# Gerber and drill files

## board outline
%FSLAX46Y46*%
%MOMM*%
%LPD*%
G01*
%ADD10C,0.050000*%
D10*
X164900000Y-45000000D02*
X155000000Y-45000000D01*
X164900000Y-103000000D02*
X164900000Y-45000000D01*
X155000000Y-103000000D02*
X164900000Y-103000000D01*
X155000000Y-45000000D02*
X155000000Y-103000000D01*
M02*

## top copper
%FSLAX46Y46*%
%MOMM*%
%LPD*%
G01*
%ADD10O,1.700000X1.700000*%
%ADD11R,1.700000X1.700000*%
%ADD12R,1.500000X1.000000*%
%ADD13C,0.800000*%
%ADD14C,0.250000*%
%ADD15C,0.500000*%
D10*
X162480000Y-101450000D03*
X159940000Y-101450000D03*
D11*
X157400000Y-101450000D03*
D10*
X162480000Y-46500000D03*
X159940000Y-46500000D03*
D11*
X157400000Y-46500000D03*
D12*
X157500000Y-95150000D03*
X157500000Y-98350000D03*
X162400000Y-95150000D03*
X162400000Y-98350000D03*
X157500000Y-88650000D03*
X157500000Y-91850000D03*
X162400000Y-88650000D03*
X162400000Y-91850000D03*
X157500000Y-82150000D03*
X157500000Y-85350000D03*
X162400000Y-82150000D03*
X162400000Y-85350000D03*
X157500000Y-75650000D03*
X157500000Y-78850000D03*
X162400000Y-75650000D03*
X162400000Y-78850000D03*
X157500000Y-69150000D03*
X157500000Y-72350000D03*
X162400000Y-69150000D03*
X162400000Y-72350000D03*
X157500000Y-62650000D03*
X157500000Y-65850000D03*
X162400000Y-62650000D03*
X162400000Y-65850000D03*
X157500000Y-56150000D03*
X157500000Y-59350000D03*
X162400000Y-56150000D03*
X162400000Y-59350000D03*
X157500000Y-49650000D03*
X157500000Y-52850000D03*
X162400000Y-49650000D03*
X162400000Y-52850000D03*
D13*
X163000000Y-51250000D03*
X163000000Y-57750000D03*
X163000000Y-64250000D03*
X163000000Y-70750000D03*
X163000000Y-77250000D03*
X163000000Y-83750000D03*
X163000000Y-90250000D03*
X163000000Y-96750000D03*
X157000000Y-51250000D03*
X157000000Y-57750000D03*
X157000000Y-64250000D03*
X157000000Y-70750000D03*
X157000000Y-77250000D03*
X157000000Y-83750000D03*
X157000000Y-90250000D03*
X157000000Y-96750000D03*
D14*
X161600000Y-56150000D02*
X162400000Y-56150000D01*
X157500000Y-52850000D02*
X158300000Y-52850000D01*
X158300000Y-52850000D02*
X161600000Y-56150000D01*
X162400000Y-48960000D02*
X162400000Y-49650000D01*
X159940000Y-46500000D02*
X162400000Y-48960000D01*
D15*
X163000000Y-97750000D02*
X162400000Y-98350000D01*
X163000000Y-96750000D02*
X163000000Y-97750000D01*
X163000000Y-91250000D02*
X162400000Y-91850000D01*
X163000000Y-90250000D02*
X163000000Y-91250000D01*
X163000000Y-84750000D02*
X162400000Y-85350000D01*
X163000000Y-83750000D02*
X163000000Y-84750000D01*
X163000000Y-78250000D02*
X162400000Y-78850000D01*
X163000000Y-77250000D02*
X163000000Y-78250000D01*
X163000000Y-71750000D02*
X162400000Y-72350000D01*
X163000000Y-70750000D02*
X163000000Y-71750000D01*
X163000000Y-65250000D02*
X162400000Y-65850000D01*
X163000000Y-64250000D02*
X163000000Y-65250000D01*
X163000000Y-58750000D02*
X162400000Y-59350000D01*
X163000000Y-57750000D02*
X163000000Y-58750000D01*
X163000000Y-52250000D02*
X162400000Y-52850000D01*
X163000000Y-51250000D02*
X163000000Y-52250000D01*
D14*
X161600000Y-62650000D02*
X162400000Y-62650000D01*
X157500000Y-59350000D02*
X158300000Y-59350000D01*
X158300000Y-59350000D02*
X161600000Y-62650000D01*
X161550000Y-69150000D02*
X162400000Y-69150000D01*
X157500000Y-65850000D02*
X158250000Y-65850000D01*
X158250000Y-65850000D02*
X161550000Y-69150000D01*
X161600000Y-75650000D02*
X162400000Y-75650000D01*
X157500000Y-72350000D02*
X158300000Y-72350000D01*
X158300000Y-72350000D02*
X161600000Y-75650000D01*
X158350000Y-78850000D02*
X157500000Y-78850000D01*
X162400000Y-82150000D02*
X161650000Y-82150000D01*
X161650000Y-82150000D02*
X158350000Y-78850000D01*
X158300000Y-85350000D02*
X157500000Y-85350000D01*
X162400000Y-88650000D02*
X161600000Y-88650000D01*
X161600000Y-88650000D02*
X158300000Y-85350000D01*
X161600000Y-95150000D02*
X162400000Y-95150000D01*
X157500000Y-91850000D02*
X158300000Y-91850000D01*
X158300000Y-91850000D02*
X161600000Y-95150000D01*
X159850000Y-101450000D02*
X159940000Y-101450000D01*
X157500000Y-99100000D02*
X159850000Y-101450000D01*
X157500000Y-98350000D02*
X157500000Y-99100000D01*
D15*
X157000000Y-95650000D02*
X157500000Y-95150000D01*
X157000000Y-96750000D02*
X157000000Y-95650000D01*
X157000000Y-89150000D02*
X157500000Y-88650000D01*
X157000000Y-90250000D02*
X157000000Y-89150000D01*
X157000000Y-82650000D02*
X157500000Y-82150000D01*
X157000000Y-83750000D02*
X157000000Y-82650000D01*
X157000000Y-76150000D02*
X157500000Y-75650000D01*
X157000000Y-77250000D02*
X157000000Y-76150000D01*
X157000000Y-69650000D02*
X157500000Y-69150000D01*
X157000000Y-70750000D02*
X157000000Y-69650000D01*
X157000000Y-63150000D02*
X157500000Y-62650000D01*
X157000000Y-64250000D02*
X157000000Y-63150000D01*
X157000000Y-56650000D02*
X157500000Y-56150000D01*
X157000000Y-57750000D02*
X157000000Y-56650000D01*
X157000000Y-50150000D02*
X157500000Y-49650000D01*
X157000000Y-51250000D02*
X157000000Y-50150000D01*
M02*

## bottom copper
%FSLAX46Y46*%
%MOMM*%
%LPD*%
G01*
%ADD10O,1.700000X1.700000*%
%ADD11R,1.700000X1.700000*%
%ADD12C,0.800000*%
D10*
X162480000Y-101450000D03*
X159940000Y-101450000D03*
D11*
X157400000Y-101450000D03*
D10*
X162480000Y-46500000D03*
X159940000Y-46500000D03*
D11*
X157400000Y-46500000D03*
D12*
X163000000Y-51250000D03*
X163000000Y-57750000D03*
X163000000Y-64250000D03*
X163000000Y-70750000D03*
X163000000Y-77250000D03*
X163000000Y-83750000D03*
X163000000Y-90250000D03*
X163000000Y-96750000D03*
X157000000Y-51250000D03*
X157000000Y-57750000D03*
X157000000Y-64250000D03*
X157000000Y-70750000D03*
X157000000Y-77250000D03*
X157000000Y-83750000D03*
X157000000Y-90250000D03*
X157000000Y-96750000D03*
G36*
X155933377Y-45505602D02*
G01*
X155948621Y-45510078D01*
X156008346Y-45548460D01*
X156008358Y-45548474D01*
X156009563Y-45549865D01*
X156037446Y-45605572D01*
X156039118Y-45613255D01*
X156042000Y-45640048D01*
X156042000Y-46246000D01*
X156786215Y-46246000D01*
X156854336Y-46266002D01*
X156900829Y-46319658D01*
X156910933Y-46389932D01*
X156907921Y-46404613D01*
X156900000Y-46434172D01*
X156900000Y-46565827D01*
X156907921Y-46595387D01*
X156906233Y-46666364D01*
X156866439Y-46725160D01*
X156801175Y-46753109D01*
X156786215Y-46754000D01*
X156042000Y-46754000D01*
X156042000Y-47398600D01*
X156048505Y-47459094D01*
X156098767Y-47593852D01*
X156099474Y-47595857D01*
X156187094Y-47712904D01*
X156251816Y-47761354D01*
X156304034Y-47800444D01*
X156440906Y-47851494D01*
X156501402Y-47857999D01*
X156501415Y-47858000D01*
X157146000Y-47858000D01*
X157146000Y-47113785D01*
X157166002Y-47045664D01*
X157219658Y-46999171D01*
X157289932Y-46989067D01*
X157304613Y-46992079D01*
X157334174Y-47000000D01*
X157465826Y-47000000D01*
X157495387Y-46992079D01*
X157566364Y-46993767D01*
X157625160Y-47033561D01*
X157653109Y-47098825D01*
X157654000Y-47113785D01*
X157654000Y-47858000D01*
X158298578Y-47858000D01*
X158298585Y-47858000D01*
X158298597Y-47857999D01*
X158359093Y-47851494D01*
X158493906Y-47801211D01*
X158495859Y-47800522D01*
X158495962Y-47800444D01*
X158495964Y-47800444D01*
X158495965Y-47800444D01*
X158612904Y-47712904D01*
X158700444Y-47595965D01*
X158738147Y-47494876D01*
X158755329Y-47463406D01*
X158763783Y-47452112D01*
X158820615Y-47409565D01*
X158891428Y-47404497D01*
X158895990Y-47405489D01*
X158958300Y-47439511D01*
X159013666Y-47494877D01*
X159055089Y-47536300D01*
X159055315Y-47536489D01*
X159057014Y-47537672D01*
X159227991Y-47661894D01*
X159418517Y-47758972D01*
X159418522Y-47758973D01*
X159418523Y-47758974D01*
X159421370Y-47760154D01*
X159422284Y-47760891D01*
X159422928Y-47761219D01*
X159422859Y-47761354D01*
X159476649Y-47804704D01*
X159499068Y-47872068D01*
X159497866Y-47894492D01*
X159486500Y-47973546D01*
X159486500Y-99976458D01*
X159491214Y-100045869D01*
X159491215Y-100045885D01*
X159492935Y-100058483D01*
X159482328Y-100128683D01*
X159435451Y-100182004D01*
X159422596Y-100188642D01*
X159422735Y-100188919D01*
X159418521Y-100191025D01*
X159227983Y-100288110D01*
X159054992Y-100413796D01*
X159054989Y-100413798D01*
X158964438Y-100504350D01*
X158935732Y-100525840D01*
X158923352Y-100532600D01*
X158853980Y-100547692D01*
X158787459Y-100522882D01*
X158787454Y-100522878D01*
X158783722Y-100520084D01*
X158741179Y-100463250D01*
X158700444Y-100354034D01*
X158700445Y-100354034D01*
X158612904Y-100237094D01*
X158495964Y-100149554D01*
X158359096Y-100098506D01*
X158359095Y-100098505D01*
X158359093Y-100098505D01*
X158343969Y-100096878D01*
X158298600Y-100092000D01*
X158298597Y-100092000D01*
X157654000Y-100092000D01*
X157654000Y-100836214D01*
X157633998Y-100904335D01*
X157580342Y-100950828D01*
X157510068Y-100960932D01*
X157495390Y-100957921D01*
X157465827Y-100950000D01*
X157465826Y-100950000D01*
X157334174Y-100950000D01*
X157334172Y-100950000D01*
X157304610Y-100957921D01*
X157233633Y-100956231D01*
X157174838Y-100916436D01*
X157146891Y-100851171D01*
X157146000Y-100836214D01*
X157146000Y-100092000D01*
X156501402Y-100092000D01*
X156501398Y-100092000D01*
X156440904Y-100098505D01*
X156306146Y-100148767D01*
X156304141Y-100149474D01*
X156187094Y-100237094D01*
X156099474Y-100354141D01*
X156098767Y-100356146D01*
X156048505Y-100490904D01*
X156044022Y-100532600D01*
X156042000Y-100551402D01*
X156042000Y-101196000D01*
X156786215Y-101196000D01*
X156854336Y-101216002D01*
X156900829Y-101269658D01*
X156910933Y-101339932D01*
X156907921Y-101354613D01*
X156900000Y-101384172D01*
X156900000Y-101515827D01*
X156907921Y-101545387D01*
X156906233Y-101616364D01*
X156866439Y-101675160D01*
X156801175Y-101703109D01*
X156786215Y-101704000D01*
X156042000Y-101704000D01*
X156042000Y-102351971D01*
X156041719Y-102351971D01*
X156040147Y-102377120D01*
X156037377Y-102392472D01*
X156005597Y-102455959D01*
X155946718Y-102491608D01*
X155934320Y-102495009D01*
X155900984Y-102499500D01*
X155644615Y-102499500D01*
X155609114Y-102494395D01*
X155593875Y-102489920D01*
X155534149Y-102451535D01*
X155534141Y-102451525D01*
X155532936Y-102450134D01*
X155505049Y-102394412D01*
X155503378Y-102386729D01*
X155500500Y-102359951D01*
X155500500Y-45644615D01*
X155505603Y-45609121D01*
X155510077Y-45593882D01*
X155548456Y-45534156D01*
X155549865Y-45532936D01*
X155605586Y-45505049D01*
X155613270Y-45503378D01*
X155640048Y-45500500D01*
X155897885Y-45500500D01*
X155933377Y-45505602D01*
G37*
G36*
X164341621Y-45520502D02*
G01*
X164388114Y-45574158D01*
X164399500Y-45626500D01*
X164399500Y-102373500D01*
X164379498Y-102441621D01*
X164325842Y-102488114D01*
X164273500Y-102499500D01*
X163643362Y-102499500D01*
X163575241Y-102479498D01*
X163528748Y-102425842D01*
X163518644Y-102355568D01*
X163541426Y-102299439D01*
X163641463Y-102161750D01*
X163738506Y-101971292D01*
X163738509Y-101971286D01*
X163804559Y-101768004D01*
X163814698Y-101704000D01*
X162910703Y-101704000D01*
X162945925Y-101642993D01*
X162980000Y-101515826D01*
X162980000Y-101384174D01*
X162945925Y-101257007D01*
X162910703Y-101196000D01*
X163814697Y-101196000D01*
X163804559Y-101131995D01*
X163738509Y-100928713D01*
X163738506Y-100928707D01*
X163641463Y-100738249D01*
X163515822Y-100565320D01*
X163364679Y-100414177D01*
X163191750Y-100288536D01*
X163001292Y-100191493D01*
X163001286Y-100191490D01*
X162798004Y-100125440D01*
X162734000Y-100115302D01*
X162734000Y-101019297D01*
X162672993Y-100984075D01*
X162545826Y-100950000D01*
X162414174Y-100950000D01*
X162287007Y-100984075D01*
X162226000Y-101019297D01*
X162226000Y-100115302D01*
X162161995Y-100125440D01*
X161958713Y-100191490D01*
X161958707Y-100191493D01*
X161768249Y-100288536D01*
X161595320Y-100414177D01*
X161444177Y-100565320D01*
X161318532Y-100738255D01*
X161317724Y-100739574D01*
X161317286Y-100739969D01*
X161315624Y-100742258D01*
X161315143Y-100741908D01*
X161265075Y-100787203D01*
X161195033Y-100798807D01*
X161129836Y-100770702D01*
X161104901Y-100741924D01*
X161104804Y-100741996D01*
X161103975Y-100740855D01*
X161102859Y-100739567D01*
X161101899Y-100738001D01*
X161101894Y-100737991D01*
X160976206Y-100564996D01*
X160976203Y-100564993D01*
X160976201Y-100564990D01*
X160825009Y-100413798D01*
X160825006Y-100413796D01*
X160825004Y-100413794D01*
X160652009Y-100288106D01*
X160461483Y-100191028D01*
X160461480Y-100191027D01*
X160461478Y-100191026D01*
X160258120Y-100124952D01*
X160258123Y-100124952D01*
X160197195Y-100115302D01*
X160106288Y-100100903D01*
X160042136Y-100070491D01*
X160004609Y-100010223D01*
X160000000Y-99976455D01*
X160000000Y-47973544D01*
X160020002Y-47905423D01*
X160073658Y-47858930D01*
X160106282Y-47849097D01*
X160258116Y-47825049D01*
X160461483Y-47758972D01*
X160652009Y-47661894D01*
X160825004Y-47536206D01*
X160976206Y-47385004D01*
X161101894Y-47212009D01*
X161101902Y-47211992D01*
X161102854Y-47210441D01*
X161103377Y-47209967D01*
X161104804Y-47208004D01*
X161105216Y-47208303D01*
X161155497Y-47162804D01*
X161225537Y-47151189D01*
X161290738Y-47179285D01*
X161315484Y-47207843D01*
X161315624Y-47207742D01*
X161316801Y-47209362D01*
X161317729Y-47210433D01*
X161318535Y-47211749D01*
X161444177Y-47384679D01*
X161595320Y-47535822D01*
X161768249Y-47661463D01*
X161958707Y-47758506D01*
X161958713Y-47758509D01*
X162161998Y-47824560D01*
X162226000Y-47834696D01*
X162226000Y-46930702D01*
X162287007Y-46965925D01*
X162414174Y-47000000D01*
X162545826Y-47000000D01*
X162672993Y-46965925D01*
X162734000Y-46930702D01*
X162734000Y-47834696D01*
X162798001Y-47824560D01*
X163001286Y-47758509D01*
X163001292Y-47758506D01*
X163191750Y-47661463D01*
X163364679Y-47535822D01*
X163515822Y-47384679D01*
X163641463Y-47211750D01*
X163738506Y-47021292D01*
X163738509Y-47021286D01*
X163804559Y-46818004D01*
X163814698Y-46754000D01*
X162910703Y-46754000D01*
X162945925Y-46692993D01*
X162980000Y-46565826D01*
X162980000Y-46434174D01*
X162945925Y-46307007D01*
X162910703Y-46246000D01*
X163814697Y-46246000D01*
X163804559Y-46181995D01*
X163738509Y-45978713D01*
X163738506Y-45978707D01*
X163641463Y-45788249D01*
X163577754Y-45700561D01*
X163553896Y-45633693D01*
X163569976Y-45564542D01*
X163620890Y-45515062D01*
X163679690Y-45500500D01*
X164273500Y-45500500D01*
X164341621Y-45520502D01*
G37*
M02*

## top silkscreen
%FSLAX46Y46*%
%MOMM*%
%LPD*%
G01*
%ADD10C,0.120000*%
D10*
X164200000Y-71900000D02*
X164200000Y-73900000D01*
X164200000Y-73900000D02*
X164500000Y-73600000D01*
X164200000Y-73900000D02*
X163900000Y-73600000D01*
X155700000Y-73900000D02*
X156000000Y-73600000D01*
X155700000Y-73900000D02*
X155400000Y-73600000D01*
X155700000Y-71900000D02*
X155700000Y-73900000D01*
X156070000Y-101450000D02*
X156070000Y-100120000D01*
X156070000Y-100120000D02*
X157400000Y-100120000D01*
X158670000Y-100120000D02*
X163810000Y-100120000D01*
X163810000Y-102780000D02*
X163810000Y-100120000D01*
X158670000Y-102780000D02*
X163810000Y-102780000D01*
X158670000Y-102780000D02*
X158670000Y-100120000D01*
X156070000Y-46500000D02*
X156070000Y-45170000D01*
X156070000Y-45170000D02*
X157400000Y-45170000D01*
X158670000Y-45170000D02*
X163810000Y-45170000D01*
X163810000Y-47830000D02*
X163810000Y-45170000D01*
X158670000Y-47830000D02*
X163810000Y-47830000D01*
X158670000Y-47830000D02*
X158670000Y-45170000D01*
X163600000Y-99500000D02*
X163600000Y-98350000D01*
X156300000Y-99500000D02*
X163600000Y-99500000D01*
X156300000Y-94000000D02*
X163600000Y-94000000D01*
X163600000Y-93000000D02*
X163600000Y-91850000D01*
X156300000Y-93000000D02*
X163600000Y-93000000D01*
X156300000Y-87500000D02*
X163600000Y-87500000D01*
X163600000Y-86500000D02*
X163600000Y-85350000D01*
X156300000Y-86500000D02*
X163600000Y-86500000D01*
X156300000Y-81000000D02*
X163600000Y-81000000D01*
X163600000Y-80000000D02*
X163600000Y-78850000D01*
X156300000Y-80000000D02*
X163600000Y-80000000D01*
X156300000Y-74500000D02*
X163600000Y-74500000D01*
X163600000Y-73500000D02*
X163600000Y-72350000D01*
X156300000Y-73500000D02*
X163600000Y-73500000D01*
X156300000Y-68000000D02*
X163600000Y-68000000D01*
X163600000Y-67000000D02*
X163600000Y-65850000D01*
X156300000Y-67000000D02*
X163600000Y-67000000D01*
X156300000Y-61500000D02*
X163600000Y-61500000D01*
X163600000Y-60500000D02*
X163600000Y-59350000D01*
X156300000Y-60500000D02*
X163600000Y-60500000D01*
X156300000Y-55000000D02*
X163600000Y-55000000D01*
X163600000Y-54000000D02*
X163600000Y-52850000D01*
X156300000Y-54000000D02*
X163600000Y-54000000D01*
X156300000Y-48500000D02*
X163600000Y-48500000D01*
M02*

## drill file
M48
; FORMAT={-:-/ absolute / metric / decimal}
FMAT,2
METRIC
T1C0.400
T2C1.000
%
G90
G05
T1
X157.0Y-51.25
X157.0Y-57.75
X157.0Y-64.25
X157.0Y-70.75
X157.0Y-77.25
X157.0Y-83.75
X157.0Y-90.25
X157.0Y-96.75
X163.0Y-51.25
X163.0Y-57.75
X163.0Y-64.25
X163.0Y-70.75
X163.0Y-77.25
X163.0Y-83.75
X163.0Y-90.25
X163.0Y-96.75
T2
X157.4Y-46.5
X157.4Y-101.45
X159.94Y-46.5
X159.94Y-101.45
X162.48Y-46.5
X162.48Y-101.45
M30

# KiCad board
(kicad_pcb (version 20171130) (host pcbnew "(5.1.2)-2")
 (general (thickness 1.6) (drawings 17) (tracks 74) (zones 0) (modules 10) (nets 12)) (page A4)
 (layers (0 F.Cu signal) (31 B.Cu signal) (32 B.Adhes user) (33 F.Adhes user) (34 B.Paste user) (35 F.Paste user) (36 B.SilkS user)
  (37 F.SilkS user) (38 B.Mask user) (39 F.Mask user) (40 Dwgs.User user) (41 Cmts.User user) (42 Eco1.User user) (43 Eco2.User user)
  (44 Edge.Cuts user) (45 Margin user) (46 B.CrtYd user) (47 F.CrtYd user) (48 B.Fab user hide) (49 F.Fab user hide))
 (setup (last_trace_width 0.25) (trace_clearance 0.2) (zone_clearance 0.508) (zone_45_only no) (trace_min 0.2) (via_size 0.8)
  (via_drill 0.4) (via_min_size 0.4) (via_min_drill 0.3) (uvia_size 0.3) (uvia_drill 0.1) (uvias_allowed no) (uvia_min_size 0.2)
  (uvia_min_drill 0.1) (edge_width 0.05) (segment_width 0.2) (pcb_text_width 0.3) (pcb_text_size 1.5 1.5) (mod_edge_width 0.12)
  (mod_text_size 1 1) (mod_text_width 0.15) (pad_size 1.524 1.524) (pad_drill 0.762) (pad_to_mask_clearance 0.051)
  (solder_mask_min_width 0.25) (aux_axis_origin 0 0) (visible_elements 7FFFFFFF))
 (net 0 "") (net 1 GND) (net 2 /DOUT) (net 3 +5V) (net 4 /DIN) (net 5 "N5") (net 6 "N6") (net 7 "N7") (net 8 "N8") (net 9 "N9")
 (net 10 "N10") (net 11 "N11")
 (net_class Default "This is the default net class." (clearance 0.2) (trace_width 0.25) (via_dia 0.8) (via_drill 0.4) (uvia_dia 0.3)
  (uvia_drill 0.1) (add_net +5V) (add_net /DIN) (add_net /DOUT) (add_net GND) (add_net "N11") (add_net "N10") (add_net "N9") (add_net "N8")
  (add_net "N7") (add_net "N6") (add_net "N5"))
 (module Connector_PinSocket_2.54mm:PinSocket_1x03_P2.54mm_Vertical (layer F.Cu) (at 157.4 101.45 90)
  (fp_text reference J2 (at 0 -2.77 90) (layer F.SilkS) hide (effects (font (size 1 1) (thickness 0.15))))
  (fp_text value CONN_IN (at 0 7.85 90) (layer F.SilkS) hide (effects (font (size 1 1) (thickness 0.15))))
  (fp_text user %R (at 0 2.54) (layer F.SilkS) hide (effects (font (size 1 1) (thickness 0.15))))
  (fp_line (start 0 -1.33) (end 1.33 -1.33) (layer F.SilkS) (width 0.12))
  (fp_line (start 1.33 -1.33) (end 1.33 0) (layer F.SilkS) (width 0.12))
  (fp_line (start 1.33 1.27) (end 1.33 6.41) (layer F.SilkS) (width 0.12))
  (fp_line (start -1.33 6.41) (end 1.33 6.41) (layer F.SilkS) (width 0.12))
  (fp_line (start -1.33 1.27) (end -1.33 6.41) (layer F.SilkS) (width 0.12))
  (fp_line (start -1.33 1.27) (end 1.33 1.27) (layer F.SilkS) (width 0.12))
  (pad 3 thru_hole oval (at 0 5.08 90) (size 1.7 1.7) (drill 1) (layers *.Cu *.Mask) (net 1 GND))
  (pad 2 thru_hole oval (at 0 2.54 90) (size 1.7 1.7) (drill 1) (layers *.Cu *.Mask) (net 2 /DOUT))
  (pad 1 thru_hole rect (at 0 0 90) (size 1.7 1.7) (drill 1) (layers *.Cu *.Mask) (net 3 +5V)))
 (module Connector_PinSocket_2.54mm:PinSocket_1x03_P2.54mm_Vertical (layer F.Cu) (at 157.4 46.5 90)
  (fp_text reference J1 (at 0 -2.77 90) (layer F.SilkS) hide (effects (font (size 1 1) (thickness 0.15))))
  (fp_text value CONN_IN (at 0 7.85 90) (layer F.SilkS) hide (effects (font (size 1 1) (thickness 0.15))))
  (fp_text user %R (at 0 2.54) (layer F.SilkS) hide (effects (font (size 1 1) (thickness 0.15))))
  (fp_line (start 0 -1.33) (end 1.33 -1.33) (layer F.SilkS) (width 0.12))
  (fp_line (start 1.33 -1.33) (end 1.33 0) (layer F.SilkS) (width 0.12))
  (fp_line (start 1.33 1.27) (end 1.33 6.41) (layer F.SilkS) (width 0.12))
  (fp_line (start -1.33 6.41) (end 1.33 6.41) (layer F.SilkS) (width 0.12))
  (fp_line (start -1.33 1.27) (end -1.33 6.41) (layer F.SilkS) (width 0.12))
  (fp_line (start -1.33 1.27) (end 1.33 1.27) (layer F.SilkS) (width 0.12))
  (pad 3 thru_hole oval (at 0 5.08 90) (size 1.7 1.7) (drill 1) (layers *.Cu *.Mask) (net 1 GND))
  (pad 2 thru_hole oval (at 0 2.54 90) (size 1.7 1.7) (drill 1) (layers *.Cu *.Mask) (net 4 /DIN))
  (pad 1 thru_hole rect (at 0 0 90) (size 1.7 1.7) (drill 1) (layers *.Cu *.Mask) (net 3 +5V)))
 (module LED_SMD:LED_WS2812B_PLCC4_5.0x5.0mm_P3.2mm (layer F.Cu) (at 159.95 96.75)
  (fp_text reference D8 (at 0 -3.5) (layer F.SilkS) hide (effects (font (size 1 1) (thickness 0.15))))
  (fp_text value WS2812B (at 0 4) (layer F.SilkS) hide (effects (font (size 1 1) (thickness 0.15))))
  (fp_line (start 3.65 2.75) (end 3.65 1.6) (layer F.SilkS) (width 0.12))
  (fp_line (start -3.65 2.75) (end 3.65 2.75) (layer F.SilkS) (width 0.12))
  (fp_line (start -3.65 -2.75) (end 3.65 -2.75) (layer F.SilkS) (width 0.12))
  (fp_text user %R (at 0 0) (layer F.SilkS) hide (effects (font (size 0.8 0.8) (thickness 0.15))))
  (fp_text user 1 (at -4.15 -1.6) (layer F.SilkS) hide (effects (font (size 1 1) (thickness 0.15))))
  (pad 1 smd rect (at -2.45 -1.6) (size 1.5 1) (layers F.Cu F.Paste F.Mask) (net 3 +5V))
  (pad 2 smd rect (at -2.45 1.6) (size 1.5 1) (layers F.Cu F.Paste F.Mask) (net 2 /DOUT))
  (pad 4 smd rect (at 2.45 -1.6) (size 1.5 1) (layers F.Cu F.Paste F.Mask) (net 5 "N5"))
  (pad 3 smd rect (at 2.45 1.6) (size 1.5 1) (layers F.Cu F.Paste F.Mask) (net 1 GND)))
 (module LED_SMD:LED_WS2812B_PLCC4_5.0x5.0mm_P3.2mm (layer F.Cu) (at 159.95 90.25)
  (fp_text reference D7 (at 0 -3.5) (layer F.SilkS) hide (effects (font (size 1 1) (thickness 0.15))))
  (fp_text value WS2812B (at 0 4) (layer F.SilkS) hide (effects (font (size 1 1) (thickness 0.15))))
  (fp_line (start 3.65 2.75) (end 3.65 1.6) (layer F.SilkS) (width 0.12))
  (fp_line (start -3.65 2.75) (end 3.65 2.75) (layer F.SilkS) (width 0.12))
  (fp_line (start -3.65 -2.75) (end 3.65 -2.75) (layer F.SilkS) (width 0.12))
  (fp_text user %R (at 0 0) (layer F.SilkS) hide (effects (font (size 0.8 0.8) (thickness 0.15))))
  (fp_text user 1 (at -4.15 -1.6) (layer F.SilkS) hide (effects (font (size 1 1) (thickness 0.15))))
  (pad 1 smd rect (at -2.45 -1.6) (size 1.5 1) (layers F.Cu F.Paste F.Mask) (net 3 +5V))
  (pad 2 smd rect (at -2.45 1.6) (size 1.5 1) (layers F.Cu F.Paste F.Mask) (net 5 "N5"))
  (pad 4 smd rect (at 2.45 -1.6) (size 1.5 1) (layers F.Cu F.Paste F.Mask) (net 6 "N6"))
  (pad 3 smd rect (at 2.45 1.6) (size 1.5 1) (layers F.Cu F.Paste F.Mask) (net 1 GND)))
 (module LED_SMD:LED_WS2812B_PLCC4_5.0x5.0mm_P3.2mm (layer F.Cu) (at 159.95 83.75)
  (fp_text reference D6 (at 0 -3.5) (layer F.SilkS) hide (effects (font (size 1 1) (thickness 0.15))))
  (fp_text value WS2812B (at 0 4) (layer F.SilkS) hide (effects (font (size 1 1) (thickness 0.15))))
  (fp_line (start 3.65 2.75) (end 3.65 1.6) (layer F.SilkS) (width 0.12))
  (fp_line (start -3.65 2.75) (end 3.65 2.75) (layer F.SilkS) (width 0.12))
  (fp_line (start -3.65 -2.75) (end 3.65 -2.75) (layer F.SilkS) (width 0.12))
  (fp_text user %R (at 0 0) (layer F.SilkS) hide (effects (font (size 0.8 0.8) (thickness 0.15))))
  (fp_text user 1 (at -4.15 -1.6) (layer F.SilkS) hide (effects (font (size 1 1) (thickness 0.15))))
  (pad 1 smd rect (at -2.45 -1.6) (size 1.5 1) (layers F.Cu F.Paste F.Mask) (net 3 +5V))
  (pad 2 smd rect (at -2.45 1.6) (size 1.5 1) (layers F.Cu F.Paste F.Mask) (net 6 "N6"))
  (pad 4 smd rect (at 2.45 -1.6) (size 1.5 1) (layers F.Cu F.Paste F.Mask) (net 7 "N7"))
  (pad 3 smd rect (at 2.45 1.6) (size 1.5 1) (layers F.Cu F.Paste F.Mask) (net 1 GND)))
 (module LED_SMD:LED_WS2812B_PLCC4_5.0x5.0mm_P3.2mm (layer F.Cu) (at 159.95 77.25)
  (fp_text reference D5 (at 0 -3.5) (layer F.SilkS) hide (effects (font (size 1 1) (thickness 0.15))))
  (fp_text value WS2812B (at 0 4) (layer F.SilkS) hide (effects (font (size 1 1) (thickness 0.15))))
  (fp_line (start 3.65 2.75) (end 3.65 1.6) (layer F.SilkS) (width 0.12))
  (fp_line (start -3.65 2.75) (end 3.65 2.75) (layer F.SilkS) (width 0.12))
  (fp_line (start -3.65 -2.75) (end 3.65 -2.75) (layer F.SilkS) (width 0.12))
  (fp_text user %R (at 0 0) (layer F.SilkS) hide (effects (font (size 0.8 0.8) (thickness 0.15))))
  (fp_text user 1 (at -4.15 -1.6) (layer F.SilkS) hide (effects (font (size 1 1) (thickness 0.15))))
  (pad 1 smd rect (at -2.45 -1.6) (size 1.5 1) (layers F.Cu F.Paste F.Mask) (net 3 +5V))
  (pad 2 smd rect (at -2.45 1.6) (size 1.5 1) (layers F.Cu F.Paste F.Mask) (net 7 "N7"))
  (pad 4 smd rect (at 2.45 -1.6) (size 1.5 1) (layers F.Cu F.Paste F.Mask) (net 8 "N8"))
  (pad 3 smd rect (at 2.45 1.6) (size 1.5 1) (layers F.Cu F.Paste F.Mask) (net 1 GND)))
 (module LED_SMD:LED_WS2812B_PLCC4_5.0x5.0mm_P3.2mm (layer F.Cu) (at 159.95 70.75)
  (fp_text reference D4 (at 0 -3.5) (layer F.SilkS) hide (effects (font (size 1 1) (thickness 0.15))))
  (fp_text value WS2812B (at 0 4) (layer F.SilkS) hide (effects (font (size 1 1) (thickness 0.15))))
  (fp_line (start 3.65 2.75) (end 3.65 1.6) (layer F.SilkS) (width 0.12))
  (fp_line (start -3.65 2.75) (end 3.65 2.75) (layer F.SilkS) (width 0.12))
  (fp_line (start -3.65 -2.75) (end 3.65 -2.75) (layer F.SilkS) (width 0.12))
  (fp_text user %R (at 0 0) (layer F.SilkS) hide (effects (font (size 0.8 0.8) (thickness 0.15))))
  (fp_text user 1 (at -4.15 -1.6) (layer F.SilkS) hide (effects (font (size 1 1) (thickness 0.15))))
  (pad 1 smd rect (at -2.45 -1.6) (size 1.5 1) (layers F.Cu F.Paste F.Mask) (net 3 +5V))
  (pad 2 smd rect (at -2.45 1.6) (size 1.5 1) (layers F.Cu F.Paste F.Mask) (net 8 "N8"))
  (pad 4 smd rect (at 2.45 -1.6) (size 1.5 1) (layers F.Cu F.Paste F.Mask) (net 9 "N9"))
  (pad 3 smd rect (at 2.45 1.6) (size 1.5 1) (layers F.Cu F.Paste F.Mask) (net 1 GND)))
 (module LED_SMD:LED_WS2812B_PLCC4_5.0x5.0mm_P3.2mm (layer F.Cu) (at 159.95 64.25)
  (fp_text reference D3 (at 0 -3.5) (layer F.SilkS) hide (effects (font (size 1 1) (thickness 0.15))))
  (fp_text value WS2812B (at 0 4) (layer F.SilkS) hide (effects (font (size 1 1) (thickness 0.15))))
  (fp_line (start 3.65 2.75) (end 3.65 1.6) (layer F.SilkS) (width 0.12))
  (fp_line (start -3.65 2.75) (end 3.65 2.75) (layer F.SilkS) (width 0.12))
  (fp_line (start -3.65 -2.75) (end 3.65 -2.75) (layer F.SilkS) (width 0.12))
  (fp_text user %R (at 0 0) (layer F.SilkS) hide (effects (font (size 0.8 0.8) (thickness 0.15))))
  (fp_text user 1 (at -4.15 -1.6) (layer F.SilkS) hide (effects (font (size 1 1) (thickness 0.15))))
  (pad 1 smd rect (at -2.45 -1.6) (size 1.5 1) (layers F.Cu F.Paste F.Mask) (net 3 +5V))
  (pad 2 smd rect (at -2.45 1.6) (size 1.5 1) (layers F.Cu F.Paste F.Mask) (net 9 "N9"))
  (pad 4 smd rect (at 2.45 -1.6) (size 1.5 1) (layers F.Cu F.Paste F.Mask) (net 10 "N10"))
  (pad 3 smd rect (at 2.45 1.6) (size 1.5 1) (layers F.Cu F.Paste F.Mask) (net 1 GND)))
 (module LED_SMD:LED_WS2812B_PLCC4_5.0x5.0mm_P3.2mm (layer F.Cu) (at 159.95 57.75)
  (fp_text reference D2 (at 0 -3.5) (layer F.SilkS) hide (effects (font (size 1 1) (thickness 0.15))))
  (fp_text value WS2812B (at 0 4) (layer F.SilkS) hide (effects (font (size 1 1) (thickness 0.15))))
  (fp_line (start 3.65 2.75) (end 3.65 1.6) (layer F.SilkS) (width 0.12))
  (fp_line (start -3.65 2.75) (end 3.65 2.75) (layer F.SilkS) (width 0.12))
  (fp_line (start -3.65 -2.75) (end 3.65 -2.75) (layer F.SilkS) (width 0.12))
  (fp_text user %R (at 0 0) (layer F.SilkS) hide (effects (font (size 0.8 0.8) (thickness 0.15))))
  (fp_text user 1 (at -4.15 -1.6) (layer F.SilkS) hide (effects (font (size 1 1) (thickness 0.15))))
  (pad 1 smd rect (at -2.45 -1.6) (size 1.5 1) (layers F.Cu F.Paste F.Mask) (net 3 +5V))
  (pad 2 smd rect (at -2.45 1.6) (size 1.5 1) (layers F.Cu F.Paste F.Mask) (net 10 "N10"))
  (pad 4 smd rect (at 2.45 -1.6) (size 1.5 1) (layers F.Cu F.Paste F.Mask) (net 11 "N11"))
  (pad 3 smd rect (at 2.45 1.6) (size 1.5 1) (layers F.Cu F.Paste F.Mask) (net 1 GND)))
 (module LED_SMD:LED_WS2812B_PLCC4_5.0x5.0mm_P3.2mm (layer F.Cu) (at 159.95 51.25)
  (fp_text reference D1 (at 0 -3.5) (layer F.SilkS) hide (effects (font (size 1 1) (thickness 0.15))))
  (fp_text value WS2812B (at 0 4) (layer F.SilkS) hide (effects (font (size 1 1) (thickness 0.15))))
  (fp_line (start 3.65 2.75) (end 3.65 1.6) (layer F.SilkS) (width 0.12))
  (fp_line (start -3.65 2.75) (end 3.65 2.75) (layer F.SilkS) (width 0.12))
  (fp_line (start -3.65 -2.75) (end 3.65 -2.75) (layer F.SilkS) (width 0.12))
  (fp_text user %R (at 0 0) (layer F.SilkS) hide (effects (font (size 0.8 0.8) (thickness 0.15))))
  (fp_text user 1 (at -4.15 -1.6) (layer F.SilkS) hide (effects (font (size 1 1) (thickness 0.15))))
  (pad 1 smd rect (at -2.45 -1.6) (size 1.5 1) (layers F.Cu F.Paste F.Mask) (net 3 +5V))
  (pad 2 smd rect (at -2.45 1.6) (size 1.5 1) (layers F.Cu F.Paste F.Mask) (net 11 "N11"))
  (pad 4 smd rect (at 2.45 -1.6) (size 1.5 1) (layers F.Cu F.Paste F.Mask) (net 4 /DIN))
  (pad 3 smd rect (at 2.45 1.6) (size 1.5 1) (layers F.Cu F.Paste F.Mask) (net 1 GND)))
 (gr_line (start 164.2 71.9) (end 164.2 73.9) (layer F.SilkS) (width 0.12))
 (gr_line (start 164.2 73.9) (end 164.5 73.6) (layer F.SilkS) (width 0.12))
 (gr_line (start 164.2 73.9) (end 163.9 73.6) (layer F.SilkS) (width 0.12))
 (gr_line (start 155.7 73.9) (end 156 73.6) (layer F.SilkS) (width 0.12))
 (gr_line (start 155.7 73.9) (end 155.4 73.6) (layer F.SilkS) (width 0.12))
 (gr_line (start 155.7 71.9) (end 155.7 73.9) (layer F.SilkS) (width 0.12))
 (gr_line (start 164.9 45) (end 155 45) (layer Edge.Cuts) (width 0.05))
 (gr_line (start 164.9 103) (end 164.9 45) (layer Edge.Cuts) (width 0.05))
 (gr_line (start 155 103) (end 164.9 103) (layer Edge.Cuts) (width 0.05))
 (gr_line (start 155 45) (end 155 103) (layer Edge.Cuts) (width 0.05))
 (segment (start 161.6 56.15) (end 162.4 56.15) (width 0.25) (layer F.Cu) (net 11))
 (segment (start 157.5 52.85) (end 158.3 52.85) (width 0.25) (layer F.Cu) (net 11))
 (segment (start 158.3 52.85) (end 161.6 56.15) (width 0.25) (layer F.Cu) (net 11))
 (segment (start 162.4 48.96) (end 162.4 49.65) (width 0.25) (layer F.Cu) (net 4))
 (segment (start 159.94 46.5) (end 162.4 48.96) (width 0.25) (layer F.Cu) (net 4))
 (via (at 163 51.25) (size 0.8) (drill 0.4) (layers F.Cu B.Cu) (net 1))
 (via (at 163 57.75) (size 0.8) (drill 0.4) (layers F.Cu B.Cu) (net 1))
 (via (at 163 64.25) (size 0.8) (drill 0.4) (layers F.Cu B.Cu) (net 1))
 (via (at 163 70.75) (size 0.8) (drill 0.4) (layers F.Cu B.Cu) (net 1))
 (via (at 163 77.25) (size 0.8) (drill 0.4) (layers F.Cu B.Cu) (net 1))
 (via (at 163 83.75) (size 0.8) (drill 0.4) (layers F.Cu B.Cu) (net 1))
 (via (at 163 90.25) (size 0.8) (drill 0.4) (layers F.Cu B.Cu) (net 1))
 (via (at 163 96.75) (size 0.8) (drill 0.4) (layers F.Cu B.Cu) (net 1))
 (segment (start 163 97.75) (end 162.4 98.35) (width 0.5) (layer F.Cu) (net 1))
 (segment (start 163 96.75) (end 163 97.75) (width 0.5) (layer F.Cu) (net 1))
 (segment (start 163 91.25) (end 162.4 91.85) (width 0.5) (layer F.Cu) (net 1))
 (segment (start 163 90.25) (end 163 91.25) (width 0.5) (layer F.Cu) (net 1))
 (segment (start 163 84.75) (end 162.4 85.35) (width 0.5) (layer F.Cu) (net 1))
 (segment (start 163 83.75) (end 163 84.75) (width 0.5) (layer F.Cu) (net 1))
 (segment (start 163 78.25) (end 162.4 78.85) (width 0.5) (layer F.Cu) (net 1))
 (segment (start 163 77.25) (end 163 78.25) (width 0.5) (layer F.Cu) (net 1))
 (segment (start 163 71.75) (end 162.4 72.35) (width 0.5) (layer F.Cu) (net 1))
 (segment (start 163 70.75) (end 163 71.75) (width 0.5) (layer F.Cu) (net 1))
 (segment (start 163 65.25) (end 162.4 65.85) (width 0.5) (layer F.Cu) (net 1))
 (segment (start 163 64.25) (end 163 65.25) (width 0.5) (layer F.Cu) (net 1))
 (segment (start 163 58.75) (end 162.4 59.35) (width 0.5) (layer F.Cu) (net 1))
 (segment (start 163 57.75) (end 163 58.75) (width 0.5) (layer F.Cu) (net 1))
 (segment (start 163 52.25) (end 162.4 52.85) (width 0.5) (layer F.Cu) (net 1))
 (segment (start 163 51.25) (end 163 52.25) (width 0.5) (layer F.Cu) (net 1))
 (segment (start 161.6 62.65) (end 162.4 62.65) (width 0.25) (layer F.Cu) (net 10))
 (segment (start 157.5 59.35) (end 158.3 59.35) (width 0.25) (layer F.Cu) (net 10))
 (segment (start 158.3 59.35) (end 161.6 62.65) (width 0.25) (layer F.Cu) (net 10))
 (segment (start 161.55 69.15) (end 162.4 69.15) (width 0.25) (layer F.Cu) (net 9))
 (segment (start 157.5 65.85) (end 158.25 65.85) (width 0.25) (layer F.Cu) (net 9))
 (segment (start 158.25 65.85) (end 161.55 69.15) (width 0.25) (layer F.Cu) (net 9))
 (segment (start 161.6 75.65) (end 162.4 75.65) (width 0.25) (layer F.Cu) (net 8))
 (segment (start 157.5 72.35) (end 158.3 72.35) (width 0.25) (layer F.Cu) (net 8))
 (segment (start 158.3 72.35) (end 161.6 75.65) (width 0.25) (layer F.Cu) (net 8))
 (segment (start 158.35 78.85) (end 157.5 78.85) (width 0.25) (layer F.Cu) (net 7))
 (segment (start 162.4 82.15) (end 161.65 82.15) (width 0.25) (layer F.Cu) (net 7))
 (segment (start 161.65 82.15) (end 158.35 78.85) (width 0.25) (layer F.Cu) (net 7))
 (segment (start 158.3 85.35) (end 157.5 85.35) (width 0.25) (layer F.Cu) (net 6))
 (segment (start 162.4 88.65) (end 161.6 88.65) (width 0.25) (layer F.Cu) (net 6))
 (segment (start 161.6 88.65) (end 158.3 85.35) (width 0.25) (layer F.Cu) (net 6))
 (segment (start 161.6 95.15) (end 162.4 95.15) (width 0.25) (layer F.Cu) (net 5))
 (segment (start 157.5 91.85) (end 158.3 91.85) (width 0.25) (layer F.Cu) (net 5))
 (segment (start 158.3 91.85) (end 161.6 95.15) (width 0.25) (layer F.Cu) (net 5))
 (segment (start 159.85 101.45) (end 159.94 101.45) (width 0.25) (layer F.Cu) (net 2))
 (segment (start 157.5 99.1) (end 159.85 101.45) (width 0.25) (layer F.Cu) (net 2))
 (segment (start 157.5 98.35) (end 157.5 99.1) (width 0.25) (layer F.Cu) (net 2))
 (via (at 157 51.25) (size 0.8) (drill 0.4) (layers F.Cu B.Cu) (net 3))
 (via (at 157 57.75) (size 0.8) (drill 0.4) (layers F.Cu B.Cu) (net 3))
 (via (at 157 64.25) (size 0.8) (drill 0.4) (layers F.Cu B.Cu) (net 3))
 (via (at 157 70.75) (size 0.8) (drill 0.4) (layers F.Cu B.Cu) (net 3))
 (via (at 157 77.25) (size 0.8) (drill 0.4) (layers F.Cu B.Cu) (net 3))
 (via (at 157 83.75) (size 0.8) (drill 0.4) (layers F.Cu B.Cu) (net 3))
 (via (at 157 90.25) (size 0.8) (drill 0.4) (layers F.Cu B.Cu) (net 3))
 (via (at 157 96.75) (size 0.8) (drill 0.4) (layers F.Cu B.Cu) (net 3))
 (segment (start 157 95.65) (end 157.5 95.15) (width 0.5) (layer F.Cu) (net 3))
 (segment (start 157 96.75) (end 157 95.65) (width 0.5) (layer F.Cu) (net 3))
 (segment (start 157 89.15) (end 157.5 88.65) (width 0.5) (layer F.Cu) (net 3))
 (segment (start 157 90.25) (end 157 89.15) (width 0.5) (layer F.Cu) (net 3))
 (segment (start 157 82.65) (end 157.5 82.15) (width 0.5) (layer F.Cu) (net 3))
 (segment (start 157 83.75) (end 157 82.65) (width 0.5) (layer F.Cu) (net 3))
 (segment (start 157 76.15) (end 157.5 75.65) (width 0.5) (layer F.Cu) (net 3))
 (segment (start 157 77.25) (end 157 76.15) (width 0.5) (layer F.Cu) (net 3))
 (segment (start 157 69.65) (end 157.5 69.15) (width 0.5) (layer F.Cu) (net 3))
 (segment (start 157 70.75) (end 157 69.65) (width 0.5) (layer F.Cu) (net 3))
 (segment (start 157 63.15) (end 157.5 62.65) (width 0.5) (layer F.Cu) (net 3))
 (segment (start 157 64.25) (end 157 63.15) (width 0.5) (layer F.Cu) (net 3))
 (segment (start 157 56.65) (end 157.5 56.15) (width 0.5) (layer F.Cu) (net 3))
 (segment (start 157 57.75) (end 157 56.65) (width 0.5) (layer F.Cu) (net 3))
 (segment (start 157 50.15) (end 157.5 49.65) (width 0.5) (layer F.Cu) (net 3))
 (segment (start 157 51.25) (end 157 50.15) (width 0.5) (layer F.Cu) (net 3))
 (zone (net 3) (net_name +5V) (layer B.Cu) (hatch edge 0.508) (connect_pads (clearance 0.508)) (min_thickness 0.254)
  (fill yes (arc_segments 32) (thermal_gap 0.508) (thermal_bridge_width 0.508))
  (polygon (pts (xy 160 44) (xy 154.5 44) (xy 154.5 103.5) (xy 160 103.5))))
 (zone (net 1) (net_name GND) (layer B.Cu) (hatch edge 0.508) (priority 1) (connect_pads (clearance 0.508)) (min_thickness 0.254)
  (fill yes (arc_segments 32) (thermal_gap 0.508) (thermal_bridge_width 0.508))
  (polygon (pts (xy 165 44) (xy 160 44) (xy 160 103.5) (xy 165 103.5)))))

